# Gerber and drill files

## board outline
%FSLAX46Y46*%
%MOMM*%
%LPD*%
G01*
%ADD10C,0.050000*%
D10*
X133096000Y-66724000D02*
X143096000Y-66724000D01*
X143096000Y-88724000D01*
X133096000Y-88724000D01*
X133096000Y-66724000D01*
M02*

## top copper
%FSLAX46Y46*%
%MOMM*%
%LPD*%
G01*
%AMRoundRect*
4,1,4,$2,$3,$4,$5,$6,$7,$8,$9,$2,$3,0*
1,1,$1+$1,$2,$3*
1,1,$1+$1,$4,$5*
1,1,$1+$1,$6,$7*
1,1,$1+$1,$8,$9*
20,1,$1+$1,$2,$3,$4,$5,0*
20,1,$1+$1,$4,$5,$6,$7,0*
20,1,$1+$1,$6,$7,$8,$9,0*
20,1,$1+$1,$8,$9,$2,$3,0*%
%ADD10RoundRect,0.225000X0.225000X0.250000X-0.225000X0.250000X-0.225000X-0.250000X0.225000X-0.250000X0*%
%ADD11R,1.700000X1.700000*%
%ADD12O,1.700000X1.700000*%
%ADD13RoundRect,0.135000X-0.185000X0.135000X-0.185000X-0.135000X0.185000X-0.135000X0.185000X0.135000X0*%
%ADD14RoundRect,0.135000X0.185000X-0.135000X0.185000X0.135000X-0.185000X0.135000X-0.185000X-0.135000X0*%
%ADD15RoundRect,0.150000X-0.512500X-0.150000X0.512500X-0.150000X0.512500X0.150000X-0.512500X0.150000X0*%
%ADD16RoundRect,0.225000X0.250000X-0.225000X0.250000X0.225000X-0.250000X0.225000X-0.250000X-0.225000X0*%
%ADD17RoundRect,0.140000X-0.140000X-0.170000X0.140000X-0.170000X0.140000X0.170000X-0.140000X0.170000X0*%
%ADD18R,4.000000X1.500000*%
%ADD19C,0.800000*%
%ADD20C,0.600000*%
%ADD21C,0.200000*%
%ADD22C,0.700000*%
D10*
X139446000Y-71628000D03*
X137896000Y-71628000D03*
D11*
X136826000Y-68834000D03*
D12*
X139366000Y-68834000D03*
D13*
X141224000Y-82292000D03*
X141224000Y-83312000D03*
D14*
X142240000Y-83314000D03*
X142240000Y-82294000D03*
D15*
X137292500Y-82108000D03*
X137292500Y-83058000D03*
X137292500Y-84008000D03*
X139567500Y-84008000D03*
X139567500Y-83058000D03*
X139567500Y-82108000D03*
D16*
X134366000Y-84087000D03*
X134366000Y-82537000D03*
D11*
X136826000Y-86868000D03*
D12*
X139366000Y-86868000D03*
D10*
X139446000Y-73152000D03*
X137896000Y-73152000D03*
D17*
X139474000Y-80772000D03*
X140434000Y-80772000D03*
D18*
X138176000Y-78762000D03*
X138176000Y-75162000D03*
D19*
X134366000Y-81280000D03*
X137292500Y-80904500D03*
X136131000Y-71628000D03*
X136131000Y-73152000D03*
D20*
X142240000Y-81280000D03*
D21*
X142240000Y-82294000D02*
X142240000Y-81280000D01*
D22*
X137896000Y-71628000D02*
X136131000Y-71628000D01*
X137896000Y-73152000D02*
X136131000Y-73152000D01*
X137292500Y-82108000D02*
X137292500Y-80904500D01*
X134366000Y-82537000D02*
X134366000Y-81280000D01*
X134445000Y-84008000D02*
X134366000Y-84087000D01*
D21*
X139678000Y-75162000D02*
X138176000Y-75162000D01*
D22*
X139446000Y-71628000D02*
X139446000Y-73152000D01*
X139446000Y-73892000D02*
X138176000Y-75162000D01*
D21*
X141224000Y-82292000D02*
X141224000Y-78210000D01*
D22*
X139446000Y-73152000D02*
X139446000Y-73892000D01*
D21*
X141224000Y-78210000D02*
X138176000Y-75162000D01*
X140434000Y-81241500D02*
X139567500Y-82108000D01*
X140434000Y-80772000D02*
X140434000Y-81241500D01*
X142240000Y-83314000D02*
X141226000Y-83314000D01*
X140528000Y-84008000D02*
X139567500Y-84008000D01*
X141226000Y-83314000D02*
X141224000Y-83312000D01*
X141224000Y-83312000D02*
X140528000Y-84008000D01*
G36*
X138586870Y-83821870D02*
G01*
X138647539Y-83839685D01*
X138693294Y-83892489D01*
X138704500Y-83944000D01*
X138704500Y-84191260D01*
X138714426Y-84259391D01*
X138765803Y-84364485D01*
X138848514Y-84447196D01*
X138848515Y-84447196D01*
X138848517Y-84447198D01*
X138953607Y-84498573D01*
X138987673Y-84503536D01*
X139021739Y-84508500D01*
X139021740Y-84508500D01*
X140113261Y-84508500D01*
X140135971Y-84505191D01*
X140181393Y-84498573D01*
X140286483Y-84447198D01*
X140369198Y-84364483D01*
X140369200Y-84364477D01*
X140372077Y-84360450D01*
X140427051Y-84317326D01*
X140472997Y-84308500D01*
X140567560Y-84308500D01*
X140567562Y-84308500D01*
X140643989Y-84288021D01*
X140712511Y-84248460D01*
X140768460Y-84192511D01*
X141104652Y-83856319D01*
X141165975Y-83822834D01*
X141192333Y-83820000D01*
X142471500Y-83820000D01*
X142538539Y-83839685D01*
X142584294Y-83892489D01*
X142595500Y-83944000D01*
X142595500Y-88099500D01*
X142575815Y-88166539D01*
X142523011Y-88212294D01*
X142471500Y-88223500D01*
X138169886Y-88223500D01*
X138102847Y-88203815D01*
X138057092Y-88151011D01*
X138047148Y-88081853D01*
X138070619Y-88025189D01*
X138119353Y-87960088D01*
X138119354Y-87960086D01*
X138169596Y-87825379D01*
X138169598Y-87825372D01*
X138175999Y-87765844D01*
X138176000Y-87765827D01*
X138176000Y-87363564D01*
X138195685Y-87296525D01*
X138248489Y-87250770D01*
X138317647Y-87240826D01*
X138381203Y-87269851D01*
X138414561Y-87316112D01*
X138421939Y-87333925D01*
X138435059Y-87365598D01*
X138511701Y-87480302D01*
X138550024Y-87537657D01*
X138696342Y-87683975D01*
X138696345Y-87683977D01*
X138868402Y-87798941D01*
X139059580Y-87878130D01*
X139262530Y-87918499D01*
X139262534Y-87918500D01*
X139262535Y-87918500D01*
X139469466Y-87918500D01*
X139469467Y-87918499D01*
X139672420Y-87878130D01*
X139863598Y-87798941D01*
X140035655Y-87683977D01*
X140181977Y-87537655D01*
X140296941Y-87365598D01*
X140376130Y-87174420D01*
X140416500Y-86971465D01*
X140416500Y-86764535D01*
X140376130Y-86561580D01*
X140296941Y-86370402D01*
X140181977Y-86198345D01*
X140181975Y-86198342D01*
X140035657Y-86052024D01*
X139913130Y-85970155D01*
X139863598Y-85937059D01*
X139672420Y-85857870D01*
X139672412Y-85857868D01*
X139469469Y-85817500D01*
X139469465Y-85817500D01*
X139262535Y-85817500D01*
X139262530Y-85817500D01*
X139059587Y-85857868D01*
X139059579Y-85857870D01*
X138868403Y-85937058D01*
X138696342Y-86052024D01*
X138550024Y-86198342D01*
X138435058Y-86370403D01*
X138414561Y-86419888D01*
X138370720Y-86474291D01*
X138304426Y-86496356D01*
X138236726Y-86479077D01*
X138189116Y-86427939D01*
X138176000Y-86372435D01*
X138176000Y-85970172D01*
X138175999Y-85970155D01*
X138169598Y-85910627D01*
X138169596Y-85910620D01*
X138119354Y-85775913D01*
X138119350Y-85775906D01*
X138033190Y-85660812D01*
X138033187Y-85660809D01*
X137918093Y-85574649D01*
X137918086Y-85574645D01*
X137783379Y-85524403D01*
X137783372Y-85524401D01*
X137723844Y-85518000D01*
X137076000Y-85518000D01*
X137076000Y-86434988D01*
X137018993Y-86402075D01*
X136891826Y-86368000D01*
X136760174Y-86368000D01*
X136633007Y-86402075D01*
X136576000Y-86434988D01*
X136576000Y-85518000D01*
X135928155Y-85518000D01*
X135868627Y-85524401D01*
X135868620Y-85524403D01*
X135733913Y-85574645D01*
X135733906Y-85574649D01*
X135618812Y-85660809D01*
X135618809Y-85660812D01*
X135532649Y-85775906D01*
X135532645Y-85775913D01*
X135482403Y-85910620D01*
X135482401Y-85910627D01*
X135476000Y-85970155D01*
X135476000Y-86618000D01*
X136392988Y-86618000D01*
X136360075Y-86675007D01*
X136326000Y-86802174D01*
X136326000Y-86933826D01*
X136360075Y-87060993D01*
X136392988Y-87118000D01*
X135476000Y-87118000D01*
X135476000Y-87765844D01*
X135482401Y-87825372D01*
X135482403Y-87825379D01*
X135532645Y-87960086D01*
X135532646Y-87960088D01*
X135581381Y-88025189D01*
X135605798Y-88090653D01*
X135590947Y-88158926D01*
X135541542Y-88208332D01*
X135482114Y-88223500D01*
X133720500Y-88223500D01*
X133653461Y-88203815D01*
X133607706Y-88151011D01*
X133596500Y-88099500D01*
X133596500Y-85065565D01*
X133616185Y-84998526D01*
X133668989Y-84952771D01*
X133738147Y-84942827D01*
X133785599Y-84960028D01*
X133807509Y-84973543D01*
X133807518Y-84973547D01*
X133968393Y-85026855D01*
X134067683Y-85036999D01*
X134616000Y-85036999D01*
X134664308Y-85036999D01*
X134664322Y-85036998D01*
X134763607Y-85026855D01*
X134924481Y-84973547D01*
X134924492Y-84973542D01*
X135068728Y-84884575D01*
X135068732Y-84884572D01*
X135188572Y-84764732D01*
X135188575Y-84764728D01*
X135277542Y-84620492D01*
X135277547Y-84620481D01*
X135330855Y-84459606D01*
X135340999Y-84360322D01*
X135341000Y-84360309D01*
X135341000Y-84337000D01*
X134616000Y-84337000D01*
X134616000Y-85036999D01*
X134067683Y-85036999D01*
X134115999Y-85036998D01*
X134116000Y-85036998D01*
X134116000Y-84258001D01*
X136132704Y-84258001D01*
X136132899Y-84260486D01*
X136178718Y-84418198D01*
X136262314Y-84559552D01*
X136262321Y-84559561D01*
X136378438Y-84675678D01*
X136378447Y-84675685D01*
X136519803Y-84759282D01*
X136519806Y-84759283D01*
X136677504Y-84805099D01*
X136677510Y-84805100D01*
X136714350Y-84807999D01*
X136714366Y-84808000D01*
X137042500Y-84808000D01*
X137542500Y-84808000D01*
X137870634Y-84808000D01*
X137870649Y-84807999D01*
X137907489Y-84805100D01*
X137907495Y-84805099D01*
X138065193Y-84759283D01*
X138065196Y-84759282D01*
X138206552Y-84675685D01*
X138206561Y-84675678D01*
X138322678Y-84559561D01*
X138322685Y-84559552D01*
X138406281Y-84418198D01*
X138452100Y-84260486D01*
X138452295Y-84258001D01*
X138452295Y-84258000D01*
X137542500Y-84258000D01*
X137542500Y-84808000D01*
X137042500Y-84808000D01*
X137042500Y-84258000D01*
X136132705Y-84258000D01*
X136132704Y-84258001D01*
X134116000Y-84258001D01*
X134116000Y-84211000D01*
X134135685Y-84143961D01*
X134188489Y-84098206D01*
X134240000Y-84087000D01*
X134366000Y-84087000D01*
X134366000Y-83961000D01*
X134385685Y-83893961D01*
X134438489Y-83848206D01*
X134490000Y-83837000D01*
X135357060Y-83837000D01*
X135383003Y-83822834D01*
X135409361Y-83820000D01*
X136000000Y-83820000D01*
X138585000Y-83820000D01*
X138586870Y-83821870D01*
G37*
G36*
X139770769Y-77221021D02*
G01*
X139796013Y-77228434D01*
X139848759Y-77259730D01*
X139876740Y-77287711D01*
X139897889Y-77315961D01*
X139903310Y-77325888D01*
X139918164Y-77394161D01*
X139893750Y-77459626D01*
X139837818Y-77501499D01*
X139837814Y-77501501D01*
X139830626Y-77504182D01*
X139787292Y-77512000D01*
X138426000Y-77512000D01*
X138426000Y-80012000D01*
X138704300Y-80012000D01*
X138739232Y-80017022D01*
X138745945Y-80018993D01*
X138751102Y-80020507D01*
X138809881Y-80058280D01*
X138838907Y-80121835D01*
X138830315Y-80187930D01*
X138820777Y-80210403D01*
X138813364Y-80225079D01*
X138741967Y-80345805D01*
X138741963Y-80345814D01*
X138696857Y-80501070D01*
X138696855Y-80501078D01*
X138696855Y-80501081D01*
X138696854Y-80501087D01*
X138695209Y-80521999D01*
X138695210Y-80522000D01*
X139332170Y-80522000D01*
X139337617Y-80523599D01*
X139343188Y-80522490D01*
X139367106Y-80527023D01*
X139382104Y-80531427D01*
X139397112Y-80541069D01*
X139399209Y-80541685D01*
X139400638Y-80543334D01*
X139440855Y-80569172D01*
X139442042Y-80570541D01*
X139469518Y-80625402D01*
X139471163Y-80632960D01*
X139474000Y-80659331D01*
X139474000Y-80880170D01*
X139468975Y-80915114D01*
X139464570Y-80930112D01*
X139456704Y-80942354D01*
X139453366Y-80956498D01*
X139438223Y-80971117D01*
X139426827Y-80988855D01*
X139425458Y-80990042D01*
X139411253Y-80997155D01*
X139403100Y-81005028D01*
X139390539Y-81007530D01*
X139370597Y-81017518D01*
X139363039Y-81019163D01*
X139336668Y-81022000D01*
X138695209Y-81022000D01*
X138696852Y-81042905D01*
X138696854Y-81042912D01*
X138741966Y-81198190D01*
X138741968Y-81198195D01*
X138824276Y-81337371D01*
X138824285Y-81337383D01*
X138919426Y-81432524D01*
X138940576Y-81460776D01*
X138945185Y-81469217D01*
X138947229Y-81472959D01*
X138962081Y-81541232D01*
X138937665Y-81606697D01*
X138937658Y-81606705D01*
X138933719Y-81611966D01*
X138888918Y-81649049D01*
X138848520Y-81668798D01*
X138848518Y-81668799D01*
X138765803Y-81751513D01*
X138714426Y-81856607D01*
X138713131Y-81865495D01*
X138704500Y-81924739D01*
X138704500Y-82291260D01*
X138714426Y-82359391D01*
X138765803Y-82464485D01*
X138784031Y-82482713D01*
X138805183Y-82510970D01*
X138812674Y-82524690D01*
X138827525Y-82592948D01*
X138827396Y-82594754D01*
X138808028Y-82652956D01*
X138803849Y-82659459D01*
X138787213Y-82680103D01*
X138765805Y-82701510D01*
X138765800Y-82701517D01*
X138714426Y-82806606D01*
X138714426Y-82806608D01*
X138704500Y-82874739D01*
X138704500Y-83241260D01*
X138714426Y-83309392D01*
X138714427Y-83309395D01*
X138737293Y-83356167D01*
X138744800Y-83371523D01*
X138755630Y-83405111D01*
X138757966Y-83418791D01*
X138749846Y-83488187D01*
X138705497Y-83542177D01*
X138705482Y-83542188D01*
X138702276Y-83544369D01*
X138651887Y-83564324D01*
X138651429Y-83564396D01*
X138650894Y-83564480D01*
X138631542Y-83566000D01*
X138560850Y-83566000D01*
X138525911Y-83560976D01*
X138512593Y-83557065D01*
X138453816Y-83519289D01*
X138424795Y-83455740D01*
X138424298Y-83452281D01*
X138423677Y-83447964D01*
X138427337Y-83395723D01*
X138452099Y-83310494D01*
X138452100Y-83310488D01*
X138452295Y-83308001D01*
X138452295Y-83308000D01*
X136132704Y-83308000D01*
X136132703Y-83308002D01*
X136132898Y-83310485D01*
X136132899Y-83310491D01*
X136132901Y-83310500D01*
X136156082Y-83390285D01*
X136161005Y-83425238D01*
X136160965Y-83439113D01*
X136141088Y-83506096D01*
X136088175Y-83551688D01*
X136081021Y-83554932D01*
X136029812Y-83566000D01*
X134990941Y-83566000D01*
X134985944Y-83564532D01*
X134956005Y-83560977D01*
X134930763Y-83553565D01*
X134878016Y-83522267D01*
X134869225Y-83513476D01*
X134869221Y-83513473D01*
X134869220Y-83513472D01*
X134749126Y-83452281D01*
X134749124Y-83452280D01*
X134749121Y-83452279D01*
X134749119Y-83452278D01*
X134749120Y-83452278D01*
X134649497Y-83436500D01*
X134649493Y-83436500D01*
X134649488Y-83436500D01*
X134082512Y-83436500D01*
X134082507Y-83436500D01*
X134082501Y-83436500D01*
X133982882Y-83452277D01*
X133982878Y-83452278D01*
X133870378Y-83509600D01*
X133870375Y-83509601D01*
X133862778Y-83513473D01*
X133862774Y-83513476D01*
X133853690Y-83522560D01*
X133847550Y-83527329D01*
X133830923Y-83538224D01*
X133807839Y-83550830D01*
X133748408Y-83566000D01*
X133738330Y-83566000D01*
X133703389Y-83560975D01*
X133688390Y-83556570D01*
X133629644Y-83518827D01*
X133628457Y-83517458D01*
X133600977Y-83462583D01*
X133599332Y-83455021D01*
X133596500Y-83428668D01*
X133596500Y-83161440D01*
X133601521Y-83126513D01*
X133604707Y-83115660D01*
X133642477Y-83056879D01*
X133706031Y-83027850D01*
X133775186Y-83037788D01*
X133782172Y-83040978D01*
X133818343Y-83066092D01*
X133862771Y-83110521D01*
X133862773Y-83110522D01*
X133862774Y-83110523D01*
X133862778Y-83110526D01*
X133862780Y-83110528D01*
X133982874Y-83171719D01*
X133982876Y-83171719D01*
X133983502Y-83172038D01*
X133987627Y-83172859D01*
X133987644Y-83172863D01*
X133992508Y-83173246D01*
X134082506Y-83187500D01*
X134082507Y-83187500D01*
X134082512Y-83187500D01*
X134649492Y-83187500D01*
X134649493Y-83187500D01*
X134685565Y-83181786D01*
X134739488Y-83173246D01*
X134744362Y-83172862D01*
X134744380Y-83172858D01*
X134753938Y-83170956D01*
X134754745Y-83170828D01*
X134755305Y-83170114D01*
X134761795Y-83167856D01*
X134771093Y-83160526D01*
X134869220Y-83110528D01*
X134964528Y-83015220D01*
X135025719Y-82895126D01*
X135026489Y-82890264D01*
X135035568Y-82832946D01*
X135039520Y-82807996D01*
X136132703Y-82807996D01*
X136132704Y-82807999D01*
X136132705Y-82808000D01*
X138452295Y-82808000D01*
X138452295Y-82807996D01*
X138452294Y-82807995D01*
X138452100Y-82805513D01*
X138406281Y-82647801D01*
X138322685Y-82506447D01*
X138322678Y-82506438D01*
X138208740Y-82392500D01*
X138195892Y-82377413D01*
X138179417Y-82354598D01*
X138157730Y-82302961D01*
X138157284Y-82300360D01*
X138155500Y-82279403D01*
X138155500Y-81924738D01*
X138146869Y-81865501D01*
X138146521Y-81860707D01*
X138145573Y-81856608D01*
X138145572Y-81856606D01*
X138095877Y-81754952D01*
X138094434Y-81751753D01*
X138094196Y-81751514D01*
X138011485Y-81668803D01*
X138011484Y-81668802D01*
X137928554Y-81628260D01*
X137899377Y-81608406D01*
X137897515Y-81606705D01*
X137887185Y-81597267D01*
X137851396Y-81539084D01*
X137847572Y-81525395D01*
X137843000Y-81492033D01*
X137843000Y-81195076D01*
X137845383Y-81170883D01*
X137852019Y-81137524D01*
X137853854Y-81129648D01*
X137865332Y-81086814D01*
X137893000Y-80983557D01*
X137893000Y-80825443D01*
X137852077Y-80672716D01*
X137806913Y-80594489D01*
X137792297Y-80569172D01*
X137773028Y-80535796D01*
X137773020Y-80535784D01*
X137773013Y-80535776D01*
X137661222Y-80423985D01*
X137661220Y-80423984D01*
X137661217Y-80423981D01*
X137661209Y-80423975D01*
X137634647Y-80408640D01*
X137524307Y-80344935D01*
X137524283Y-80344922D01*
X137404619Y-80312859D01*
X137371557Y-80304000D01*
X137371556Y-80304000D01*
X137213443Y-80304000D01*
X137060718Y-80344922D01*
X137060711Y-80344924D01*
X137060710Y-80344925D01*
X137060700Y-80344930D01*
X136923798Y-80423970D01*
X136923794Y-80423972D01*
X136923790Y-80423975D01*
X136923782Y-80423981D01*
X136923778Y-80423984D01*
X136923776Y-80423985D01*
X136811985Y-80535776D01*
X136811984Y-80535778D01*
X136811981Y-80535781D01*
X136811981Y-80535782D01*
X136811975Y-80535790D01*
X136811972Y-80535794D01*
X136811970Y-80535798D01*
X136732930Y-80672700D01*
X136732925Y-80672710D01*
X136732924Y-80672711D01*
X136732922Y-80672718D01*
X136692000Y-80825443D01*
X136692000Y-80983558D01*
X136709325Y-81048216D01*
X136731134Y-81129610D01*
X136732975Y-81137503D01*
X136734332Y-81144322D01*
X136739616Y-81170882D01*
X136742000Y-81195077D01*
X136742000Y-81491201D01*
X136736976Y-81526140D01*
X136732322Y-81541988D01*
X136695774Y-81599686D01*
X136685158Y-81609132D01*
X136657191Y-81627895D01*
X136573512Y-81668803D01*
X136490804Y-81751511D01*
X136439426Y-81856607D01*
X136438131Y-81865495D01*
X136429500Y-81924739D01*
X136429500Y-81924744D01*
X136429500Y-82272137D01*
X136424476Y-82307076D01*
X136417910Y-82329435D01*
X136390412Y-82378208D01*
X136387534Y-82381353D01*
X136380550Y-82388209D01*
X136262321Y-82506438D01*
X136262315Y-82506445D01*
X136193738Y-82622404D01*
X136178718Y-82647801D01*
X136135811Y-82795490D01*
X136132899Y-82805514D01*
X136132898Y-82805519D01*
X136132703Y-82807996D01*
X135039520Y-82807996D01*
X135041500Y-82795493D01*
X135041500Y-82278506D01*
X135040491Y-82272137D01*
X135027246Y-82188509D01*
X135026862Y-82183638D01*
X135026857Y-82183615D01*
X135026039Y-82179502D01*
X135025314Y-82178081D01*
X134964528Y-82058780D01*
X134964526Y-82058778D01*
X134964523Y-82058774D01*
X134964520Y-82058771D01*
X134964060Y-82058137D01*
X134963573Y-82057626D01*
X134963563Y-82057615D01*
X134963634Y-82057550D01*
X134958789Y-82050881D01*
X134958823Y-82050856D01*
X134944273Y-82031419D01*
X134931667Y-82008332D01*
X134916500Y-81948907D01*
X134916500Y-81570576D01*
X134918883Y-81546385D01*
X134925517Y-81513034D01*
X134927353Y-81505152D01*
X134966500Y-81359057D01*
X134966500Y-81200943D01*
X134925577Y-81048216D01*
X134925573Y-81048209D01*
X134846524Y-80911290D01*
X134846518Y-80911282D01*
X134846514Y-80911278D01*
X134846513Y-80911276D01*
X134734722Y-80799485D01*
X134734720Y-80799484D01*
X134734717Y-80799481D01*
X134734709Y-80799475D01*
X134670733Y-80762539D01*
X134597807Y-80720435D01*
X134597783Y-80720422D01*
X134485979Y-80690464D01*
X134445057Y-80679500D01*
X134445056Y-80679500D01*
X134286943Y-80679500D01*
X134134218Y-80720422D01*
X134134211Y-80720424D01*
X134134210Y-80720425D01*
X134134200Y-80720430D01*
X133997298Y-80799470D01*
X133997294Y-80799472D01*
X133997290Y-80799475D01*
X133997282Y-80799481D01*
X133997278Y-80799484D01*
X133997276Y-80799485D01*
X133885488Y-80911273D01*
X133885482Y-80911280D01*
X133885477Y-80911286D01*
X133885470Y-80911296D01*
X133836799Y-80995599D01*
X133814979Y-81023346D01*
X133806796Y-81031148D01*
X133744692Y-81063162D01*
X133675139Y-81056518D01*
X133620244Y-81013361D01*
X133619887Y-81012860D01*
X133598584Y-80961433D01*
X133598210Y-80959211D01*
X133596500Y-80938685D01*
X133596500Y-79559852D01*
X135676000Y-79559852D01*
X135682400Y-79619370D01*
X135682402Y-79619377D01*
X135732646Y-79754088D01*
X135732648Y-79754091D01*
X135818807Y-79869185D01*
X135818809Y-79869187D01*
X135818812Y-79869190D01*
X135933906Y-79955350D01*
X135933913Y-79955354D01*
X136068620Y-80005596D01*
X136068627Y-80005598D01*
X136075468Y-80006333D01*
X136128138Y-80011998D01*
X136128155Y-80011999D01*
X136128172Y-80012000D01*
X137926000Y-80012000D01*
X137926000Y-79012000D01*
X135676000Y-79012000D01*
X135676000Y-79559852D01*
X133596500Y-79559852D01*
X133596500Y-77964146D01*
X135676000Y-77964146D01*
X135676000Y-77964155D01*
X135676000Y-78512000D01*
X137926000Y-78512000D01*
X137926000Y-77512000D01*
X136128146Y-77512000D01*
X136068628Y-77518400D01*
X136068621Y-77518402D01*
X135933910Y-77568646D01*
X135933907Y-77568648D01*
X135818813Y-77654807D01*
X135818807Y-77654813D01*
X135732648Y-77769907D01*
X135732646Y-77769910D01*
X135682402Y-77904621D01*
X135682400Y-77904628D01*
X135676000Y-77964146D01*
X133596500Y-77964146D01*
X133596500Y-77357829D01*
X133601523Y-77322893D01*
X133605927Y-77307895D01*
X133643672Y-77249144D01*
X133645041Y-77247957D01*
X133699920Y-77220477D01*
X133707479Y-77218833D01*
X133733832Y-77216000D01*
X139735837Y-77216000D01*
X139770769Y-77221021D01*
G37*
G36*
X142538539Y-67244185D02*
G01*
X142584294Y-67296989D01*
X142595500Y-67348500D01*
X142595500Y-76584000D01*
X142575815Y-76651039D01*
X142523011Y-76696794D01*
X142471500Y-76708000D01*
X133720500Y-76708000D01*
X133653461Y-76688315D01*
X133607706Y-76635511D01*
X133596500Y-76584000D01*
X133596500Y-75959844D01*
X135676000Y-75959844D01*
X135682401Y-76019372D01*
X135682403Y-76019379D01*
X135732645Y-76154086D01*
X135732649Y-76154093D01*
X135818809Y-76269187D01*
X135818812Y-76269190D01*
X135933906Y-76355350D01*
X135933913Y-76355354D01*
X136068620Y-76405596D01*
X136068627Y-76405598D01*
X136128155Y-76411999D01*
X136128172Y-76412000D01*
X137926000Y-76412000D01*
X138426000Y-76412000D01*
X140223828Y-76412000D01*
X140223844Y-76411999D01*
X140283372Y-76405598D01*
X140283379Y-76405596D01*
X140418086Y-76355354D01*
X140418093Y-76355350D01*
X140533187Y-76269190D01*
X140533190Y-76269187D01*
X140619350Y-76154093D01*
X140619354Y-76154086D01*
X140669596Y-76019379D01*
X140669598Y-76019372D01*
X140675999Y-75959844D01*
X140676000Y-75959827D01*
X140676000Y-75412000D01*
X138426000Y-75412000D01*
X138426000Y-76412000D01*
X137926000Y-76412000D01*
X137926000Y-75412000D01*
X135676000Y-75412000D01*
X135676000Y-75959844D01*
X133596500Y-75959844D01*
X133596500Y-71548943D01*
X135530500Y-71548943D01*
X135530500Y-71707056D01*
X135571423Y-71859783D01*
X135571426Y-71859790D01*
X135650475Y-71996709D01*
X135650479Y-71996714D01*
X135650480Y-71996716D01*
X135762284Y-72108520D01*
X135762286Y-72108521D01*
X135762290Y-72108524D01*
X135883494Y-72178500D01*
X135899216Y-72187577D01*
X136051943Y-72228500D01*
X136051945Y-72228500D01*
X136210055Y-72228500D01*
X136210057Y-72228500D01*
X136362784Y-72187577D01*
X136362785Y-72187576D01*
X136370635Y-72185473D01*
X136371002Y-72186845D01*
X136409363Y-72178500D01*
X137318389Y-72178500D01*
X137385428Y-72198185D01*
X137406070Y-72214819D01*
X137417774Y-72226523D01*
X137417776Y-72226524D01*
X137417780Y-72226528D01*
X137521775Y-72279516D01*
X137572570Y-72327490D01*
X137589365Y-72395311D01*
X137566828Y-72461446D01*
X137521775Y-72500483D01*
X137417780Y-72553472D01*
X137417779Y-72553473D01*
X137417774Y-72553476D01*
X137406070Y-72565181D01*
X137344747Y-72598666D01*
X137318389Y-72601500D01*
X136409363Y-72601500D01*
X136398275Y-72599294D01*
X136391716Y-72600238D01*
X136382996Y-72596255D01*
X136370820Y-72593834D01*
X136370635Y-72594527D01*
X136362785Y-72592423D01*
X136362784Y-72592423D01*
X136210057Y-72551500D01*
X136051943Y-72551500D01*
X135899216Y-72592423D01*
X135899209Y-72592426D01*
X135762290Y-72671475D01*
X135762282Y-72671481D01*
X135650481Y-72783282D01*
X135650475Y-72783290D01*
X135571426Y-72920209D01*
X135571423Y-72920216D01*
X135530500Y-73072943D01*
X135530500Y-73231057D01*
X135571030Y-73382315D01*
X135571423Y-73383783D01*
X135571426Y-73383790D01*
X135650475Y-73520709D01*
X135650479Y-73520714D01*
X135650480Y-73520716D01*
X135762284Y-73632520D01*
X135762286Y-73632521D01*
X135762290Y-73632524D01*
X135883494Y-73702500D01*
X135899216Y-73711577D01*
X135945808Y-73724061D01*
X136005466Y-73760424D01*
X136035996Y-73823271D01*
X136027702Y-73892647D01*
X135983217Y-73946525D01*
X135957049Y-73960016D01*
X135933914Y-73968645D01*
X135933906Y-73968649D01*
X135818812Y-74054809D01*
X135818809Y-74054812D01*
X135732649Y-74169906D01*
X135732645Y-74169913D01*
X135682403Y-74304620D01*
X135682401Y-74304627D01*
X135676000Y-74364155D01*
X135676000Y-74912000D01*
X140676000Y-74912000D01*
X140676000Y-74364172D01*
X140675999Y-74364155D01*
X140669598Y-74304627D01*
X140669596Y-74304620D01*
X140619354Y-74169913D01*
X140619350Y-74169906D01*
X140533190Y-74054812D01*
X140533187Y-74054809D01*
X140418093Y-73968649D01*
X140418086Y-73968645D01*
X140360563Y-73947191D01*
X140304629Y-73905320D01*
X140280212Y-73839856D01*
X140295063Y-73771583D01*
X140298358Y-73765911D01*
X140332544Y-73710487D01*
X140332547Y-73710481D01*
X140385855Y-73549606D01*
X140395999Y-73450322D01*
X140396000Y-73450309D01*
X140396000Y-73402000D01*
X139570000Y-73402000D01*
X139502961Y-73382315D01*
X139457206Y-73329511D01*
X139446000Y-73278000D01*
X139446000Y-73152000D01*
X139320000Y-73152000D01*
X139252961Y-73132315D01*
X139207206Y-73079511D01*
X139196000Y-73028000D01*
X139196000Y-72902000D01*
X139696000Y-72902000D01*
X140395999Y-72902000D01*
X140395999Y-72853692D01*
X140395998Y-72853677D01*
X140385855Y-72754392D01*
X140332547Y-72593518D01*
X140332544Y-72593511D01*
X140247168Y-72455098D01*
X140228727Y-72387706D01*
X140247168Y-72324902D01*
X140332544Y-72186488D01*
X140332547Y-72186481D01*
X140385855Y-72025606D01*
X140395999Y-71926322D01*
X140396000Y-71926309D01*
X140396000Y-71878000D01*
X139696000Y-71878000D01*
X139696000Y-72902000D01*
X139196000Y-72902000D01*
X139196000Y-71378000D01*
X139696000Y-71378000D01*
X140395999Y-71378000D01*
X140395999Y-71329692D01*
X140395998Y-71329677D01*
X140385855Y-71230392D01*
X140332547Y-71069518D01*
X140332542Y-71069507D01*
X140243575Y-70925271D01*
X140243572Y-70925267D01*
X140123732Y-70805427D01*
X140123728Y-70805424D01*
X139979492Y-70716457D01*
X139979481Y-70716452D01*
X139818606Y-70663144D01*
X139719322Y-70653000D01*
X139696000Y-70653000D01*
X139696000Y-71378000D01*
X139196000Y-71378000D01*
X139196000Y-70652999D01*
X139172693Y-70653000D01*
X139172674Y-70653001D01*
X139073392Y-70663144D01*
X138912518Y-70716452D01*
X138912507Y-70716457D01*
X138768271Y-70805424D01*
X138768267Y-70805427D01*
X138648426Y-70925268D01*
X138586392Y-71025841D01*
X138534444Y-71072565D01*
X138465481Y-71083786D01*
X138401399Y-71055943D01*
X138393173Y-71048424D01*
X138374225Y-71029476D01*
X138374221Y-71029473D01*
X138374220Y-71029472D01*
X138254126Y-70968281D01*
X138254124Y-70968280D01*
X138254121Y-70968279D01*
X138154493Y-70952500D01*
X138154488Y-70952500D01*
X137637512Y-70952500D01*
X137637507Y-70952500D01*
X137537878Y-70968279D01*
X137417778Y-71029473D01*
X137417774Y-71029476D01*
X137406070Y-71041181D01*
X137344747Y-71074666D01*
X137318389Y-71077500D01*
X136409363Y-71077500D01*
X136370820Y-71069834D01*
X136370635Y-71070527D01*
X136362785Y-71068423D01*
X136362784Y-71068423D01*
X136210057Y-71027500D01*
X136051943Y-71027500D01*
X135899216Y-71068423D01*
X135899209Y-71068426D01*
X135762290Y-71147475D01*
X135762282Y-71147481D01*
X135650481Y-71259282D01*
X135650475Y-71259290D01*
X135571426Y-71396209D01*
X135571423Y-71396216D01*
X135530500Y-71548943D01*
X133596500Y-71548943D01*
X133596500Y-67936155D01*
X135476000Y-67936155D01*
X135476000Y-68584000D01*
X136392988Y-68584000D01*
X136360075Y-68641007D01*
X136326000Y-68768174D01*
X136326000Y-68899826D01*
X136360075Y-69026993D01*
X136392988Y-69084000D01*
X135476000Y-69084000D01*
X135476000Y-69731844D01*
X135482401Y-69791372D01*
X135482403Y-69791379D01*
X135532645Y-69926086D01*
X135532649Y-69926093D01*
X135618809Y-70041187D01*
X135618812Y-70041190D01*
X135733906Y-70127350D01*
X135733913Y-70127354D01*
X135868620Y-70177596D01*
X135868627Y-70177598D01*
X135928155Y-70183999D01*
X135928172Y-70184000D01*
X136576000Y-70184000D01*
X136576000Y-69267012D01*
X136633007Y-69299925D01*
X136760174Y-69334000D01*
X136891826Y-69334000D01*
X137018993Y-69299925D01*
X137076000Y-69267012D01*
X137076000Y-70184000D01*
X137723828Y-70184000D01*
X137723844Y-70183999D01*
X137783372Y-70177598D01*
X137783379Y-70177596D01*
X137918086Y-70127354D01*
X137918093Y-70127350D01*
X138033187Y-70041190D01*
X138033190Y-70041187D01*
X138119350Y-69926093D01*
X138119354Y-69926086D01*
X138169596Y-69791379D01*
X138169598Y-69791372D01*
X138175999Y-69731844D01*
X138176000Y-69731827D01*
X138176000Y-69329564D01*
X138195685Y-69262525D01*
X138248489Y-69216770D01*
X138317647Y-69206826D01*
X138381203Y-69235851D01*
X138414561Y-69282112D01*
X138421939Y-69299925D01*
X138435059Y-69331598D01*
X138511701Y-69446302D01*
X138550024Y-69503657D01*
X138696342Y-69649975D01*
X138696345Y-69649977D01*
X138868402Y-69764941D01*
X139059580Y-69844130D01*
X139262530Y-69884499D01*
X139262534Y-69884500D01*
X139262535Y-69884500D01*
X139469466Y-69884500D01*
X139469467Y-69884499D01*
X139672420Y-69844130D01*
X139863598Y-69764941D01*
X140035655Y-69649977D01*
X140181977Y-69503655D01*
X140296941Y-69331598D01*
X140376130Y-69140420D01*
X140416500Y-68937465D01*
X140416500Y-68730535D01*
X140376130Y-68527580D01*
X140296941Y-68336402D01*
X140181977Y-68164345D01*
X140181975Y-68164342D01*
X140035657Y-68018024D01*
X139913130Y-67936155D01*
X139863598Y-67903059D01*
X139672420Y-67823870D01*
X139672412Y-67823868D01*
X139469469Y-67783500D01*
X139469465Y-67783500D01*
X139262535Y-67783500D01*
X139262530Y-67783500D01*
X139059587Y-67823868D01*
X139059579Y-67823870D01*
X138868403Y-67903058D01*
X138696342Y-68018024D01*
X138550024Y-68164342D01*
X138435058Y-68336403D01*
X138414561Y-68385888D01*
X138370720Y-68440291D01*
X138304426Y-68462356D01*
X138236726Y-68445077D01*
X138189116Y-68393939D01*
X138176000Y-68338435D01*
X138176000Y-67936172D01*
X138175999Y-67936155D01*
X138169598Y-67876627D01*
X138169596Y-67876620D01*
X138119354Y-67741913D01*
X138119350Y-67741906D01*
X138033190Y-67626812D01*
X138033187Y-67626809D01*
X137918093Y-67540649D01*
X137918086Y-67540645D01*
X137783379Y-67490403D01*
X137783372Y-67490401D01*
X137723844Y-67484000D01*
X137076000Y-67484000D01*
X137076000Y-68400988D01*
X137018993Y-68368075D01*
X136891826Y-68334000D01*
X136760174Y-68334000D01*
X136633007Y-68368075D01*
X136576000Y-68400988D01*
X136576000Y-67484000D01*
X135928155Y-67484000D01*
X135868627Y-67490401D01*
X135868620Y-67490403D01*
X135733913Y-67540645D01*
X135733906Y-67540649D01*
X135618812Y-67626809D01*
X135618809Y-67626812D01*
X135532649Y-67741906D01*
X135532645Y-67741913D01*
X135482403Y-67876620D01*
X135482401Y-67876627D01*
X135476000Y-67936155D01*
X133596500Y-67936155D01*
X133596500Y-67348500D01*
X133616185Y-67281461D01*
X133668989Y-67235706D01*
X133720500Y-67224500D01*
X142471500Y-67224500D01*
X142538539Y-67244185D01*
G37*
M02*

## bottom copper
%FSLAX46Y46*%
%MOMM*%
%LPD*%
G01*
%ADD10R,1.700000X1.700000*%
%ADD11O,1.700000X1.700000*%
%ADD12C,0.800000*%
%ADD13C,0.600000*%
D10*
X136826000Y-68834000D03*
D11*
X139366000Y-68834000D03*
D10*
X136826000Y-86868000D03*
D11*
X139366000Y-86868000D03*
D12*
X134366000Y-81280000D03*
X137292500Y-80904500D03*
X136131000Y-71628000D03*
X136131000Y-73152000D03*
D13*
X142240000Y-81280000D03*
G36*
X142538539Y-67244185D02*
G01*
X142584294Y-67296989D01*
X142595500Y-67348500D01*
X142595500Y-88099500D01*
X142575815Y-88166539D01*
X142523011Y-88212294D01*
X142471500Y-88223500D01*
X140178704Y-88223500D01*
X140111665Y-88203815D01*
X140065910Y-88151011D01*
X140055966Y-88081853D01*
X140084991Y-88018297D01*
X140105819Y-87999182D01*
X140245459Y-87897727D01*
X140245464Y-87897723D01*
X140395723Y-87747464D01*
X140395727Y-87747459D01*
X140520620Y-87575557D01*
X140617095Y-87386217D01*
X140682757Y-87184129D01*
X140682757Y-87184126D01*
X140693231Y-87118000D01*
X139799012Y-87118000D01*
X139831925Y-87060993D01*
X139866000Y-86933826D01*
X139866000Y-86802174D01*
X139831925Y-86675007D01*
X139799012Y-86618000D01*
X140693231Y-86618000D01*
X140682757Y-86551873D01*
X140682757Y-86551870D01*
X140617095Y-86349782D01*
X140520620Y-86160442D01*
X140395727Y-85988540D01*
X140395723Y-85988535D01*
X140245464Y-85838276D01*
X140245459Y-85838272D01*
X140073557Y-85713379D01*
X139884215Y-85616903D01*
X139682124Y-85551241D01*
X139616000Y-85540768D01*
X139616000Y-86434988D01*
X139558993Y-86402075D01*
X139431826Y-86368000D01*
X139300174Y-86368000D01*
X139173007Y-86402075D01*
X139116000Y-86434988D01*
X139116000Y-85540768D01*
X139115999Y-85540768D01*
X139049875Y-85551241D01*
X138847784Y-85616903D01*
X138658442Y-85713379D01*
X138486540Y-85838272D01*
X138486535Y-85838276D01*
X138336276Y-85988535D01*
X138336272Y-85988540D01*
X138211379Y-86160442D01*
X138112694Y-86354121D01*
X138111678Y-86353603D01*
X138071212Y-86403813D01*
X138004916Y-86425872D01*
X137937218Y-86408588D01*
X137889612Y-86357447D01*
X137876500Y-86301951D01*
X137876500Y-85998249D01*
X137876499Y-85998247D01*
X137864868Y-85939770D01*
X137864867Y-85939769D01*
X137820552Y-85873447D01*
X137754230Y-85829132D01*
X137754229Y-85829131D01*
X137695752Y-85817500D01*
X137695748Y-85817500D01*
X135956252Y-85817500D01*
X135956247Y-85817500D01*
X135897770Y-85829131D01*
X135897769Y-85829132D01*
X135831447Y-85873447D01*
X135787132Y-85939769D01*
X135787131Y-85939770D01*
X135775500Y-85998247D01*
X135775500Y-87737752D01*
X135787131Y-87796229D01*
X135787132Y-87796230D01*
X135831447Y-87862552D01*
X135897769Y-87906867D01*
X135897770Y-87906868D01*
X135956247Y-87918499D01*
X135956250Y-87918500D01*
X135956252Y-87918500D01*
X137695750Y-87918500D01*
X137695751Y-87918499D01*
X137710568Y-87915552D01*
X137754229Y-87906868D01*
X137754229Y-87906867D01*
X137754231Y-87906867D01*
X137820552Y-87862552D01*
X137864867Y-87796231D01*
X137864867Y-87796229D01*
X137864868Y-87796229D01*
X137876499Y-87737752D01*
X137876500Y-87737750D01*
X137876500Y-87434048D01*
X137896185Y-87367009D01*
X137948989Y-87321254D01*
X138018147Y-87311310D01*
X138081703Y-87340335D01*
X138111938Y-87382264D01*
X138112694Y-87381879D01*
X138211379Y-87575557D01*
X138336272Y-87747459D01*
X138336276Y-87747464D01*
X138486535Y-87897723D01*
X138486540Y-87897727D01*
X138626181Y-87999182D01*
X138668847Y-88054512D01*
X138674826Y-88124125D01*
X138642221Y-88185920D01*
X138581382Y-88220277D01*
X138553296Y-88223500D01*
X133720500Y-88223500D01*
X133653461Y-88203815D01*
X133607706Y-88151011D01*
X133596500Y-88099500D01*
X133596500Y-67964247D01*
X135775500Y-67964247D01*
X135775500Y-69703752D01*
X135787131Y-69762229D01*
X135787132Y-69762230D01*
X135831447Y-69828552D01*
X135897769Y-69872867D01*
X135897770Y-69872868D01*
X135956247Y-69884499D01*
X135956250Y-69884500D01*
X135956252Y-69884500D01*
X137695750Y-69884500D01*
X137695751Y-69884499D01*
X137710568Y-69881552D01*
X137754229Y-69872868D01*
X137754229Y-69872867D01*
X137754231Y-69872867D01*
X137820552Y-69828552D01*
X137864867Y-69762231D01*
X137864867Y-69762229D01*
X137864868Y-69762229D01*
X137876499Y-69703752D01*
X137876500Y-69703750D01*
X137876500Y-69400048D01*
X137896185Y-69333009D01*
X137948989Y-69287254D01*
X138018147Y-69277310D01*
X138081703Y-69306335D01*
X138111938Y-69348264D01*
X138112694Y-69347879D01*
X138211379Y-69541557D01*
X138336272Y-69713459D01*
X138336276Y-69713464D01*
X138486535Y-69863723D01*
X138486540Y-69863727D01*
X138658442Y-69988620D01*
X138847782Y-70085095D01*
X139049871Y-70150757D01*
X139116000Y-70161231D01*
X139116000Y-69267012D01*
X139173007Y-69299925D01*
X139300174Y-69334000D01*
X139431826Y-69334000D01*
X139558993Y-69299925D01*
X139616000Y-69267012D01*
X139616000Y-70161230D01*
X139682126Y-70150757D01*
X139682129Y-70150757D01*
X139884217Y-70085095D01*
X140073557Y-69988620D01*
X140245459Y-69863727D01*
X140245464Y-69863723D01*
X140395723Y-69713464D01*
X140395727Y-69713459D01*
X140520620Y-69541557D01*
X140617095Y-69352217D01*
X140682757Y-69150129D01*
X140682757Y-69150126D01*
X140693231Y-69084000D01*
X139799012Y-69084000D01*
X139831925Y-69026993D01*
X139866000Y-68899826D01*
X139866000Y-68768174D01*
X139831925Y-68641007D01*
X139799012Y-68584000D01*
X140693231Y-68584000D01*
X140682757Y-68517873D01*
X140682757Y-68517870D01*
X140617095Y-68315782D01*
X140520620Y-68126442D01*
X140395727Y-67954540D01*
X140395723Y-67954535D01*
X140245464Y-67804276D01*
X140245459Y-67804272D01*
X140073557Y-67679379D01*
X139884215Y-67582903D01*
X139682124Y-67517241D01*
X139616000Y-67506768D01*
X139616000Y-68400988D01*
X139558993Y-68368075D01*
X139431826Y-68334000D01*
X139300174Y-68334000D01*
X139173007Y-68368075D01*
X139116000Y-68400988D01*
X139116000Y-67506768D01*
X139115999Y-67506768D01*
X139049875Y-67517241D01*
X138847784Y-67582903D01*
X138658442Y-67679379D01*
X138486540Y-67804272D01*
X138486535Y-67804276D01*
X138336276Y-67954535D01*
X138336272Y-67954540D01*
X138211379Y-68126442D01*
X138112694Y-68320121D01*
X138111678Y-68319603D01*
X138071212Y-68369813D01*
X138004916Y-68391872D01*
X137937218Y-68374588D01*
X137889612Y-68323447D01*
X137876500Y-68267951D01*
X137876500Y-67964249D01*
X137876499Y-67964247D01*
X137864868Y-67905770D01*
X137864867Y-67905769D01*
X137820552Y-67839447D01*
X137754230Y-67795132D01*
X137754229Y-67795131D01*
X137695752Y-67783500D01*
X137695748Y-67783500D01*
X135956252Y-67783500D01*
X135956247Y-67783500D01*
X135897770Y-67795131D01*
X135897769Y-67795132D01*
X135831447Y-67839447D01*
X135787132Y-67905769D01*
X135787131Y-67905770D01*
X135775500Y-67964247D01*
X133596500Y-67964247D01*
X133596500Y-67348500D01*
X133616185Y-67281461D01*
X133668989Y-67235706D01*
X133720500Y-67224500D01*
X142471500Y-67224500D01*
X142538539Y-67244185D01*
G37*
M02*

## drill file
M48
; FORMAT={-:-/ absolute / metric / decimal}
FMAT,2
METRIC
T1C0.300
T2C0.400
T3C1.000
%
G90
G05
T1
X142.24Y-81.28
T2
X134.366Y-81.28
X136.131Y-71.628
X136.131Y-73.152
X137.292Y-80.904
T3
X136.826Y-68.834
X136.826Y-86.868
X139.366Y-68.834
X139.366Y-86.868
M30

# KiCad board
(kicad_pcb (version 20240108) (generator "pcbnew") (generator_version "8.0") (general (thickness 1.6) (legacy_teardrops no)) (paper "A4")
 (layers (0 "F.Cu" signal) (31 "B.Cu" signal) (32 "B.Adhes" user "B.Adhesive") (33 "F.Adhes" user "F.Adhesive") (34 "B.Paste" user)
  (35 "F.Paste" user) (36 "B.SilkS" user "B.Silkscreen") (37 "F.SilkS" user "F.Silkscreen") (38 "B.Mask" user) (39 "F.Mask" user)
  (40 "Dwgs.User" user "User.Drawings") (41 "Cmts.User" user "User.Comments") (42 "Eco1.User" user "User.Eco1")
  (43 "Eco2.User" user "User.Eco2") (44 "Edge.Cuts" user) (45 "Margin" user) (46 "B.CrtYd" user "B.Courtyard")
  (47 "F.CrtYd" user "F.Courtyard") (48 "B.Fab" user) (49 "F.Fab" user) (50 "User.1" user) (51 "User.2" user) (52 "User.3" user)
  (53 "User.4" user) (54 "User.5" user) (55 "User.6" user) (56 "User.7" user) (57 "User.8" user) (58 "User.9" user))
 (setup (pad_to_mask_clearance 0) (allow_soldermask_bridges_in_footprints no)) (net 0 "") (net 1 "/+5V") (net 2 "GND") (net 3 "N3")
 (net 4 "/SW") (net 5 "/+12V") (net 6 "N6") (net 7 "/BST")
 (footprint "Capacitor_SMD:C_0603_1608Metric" (layer "F.Cu") (at 138.671 71.628 180)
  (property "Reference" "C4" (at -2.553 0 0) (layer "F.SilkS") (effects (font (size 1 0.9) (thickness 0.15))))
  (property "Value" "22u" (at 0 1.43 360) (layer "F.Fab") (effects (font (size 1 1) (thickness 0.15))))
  (pad "1" smd roundrect (at -0.775 0 180) (size 0.9 0.95) (layers "F.Cu" "F.Paste" "F.Mask") (roundrect_rratio 0.25) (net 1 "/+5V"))
  (pad "2" smd roundrect (at 0.775 0 180) (size 0.9 0.95) (layers "F.Cu" "F.Paste" "F.Mask") (roundrect_rratio 0.25) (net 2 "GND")))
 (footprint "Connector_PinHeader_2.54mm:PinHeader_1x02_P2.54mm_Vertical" (layer "F.Cu") (at 136.826 68.834 90)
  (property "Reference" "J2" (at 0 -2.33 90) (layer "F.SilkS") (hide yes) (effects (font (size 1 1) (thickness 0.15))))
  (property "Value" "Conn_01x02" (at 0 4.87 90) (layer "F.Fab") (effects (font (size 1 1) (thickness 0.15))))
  (pad "1" thru_hole rect (at 0 0 90) (size 1.7 1.7) (drill 1) (layers "*.Cu" "*.Mask") (remove_unused_layers no) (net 1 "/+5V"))
  (pad "2" thru_hole oval (at 0 2.54 90) (size 1.7 1.7) (drill 1) (layers "*.Cu" "*.Mask") (remove_unused_layers no) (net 2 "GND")))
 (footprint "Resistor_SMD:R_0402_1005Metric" (layer "F.Cu") (at 141.224 82.802 -90)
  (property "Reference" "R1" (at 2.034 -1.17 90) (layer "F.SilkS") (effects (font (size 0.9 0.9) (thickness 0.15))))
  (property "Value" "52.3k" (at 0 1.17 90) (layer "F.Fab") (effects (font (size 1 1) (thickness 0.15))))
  (pad "1" smd roundrect (at -0.51 0 270) (size 0.54 0.64) (layers "F.Cu" "F.Paste" "F.Mask") (roundrect_rratio 0.25) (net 1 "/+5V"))
  (pad "2" smd roundrect (at 0.51 0 270) (size 0.54 0.64) (layers "F.Cu" "F.Paste" "F.Mask") (roundrect_rratio 0.25) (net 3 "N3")))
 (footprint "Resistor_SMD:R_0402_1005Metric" (layer "F.Cu") (at 142.24 82.804 90)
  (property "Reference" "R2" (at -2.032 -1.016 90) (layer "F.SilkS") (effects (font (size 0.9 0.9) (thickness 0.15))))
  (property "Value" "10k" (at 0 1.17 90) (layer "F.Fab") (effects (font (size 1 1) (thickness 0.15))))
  (pad "1" smd roundrect (at -0.51 0 90) (size 0.54 0.64) (layers "F.Cu" "F.Paste" "F.Mask") (roundrect_rratio 0.25) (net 3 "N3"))
  (pad "2" smd roundrect (at 0.51 0 90) (size 0.54 0.64) (layers "F.Cu" "F.Paste" "F.Mask") (roundrect_rratio 0.25) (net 2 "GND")))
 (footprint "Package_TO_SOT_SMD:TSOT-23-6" (layer "F.Cu") (at 138.43 83.058)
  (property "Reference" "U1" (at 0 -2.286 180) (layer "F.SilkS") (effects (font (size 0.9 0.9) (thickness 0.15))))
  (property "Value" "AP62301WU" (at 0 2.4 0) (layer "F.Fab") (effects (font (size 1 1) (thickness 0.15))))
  (pad "1" smd roundrect (at -1.1375 -0.95) (size 1.325 0.6) (layers "F.Cu" "F.Paste" "F.Mask") (roundrect_rratio 0.25) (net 2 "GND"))
  (pad "2" smd roundrect (at -1.1375 0) (size 1.325 0.6) (layers "F.Cu" "F.Paste" "F.Mask") (roundrect_rratio 0.25) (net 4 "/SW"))
  (pad "3" smd roundrect (at -1.1375 0.95) (size 1.325 0.6) (layers "F.Cu" "F.Paste" "F.Mask") (roundrect_rratio 0.25) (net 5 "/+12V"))
  (pad "4" smd roundrect (at 1.1375 0.95) (size 1.325 0.6) (layers "F.Cu" "F.Paste" "F.Mask") (roundrect_rratio 0.25) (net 3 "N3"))
  (pad "5" smd roundrect (at 1.1375 0) (size 1.325 0.6) (layers "F.Cu" "F.Paste" "F.Mask") (roundrect_rratio 0.25) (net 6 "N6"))
  (pad "6" smd roundrect (at 1.1375 -0.95) (size 1.325 0.6) (layers "F.Cu" "F.Paste" "F.Mask") (roundrect_rratio 0.25) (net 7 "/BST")))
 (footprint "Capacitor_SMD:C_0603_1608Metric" (layer "F.Cu") (at 134.366 83.312 90)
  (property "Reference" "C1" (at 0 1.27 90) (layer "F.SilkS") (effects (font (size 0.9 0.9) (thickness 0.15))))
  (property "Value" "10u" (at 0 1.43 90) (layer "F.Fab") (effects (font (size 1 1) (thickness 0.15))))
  (pad "1" smd roundrect (at -0.775 0 90) (size 0.9 0.95) (layers "F.Cu" "F.Paste" "F.Mask") (roundrect_rratio 0.25) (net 5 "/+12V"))
  (pad "2" smd roundrect (at 0.775 0 90) (size 0.9 0.95) (layers "F.Cu" "F.Paste" "F.Mask") (roundrect_rratio 0.25) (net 2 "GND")))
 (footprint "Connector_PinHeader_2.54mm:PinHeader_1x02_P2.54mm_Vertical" (layer "F.Cu") (at 136.826 86.868 90)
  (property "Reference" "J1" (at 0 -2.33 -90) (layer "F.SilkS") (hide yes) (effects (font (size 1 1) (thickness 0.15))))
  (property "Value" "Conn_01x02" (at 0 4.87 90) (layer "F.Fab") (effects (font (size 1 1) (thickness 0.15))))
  (pad "1" thru_hole rect (at 0 0 90) (size 1.7 1.7) (drill 1) (layers "*.Cu" "*.Mask") (remove_unused_layers no) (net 5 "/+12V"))
  (pad "2" thru_hole oval (at 0 2.54 90) (size 1.7 1.7) (drill 1) (layers "*.Cu" "*.Mask") (remove_unused_layers no) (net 2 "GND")))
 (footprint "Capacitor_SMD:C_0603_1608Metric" (layer "F.Cu") (at 138.671 73.152 180)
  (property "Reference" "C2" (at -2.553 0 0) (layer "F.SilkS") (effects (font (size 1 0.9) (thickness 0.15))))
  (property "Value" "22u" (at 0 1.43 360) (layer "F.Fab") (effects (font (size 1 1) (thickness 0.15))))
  (pad "1" smd roundrect (at -0.775 0 180) (size 0.9 0.95) (layers "F.Cu" "F.Paste" "F.Mask") (roundrect_rratio 0.25) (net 1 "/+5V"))
  (pad "2" smd roundrect (at 0.775 0 180) (size 0.9 0.95) (layers "F.Cu" "F.Paste" "F.Mask") (roundrect_rratio 0.25) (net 2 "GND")))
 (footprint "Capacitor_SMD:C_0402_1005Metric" (layer "F.Cu") (at 139.954 80.772)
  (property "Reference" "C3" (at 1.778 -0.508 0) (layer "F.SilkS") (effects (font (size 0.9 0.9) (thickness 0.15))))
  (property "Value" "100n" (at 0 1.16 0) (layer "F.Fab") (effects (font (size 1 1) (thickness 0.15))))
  (pad "1" smd roundrect (at -0.48 0) (size 0.56 0.62) (layers "F.Cu" "F.Paste" "F.Mask") (roundrect_rratio 0.25) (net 4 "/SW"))
  (pad "2" smd roundrect (at 0.48 0) (size 0.56 0.62) (layers "F.Cu" "F.Paste" "F.Mask") (roundrect_rratio 0.25) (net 7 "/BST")))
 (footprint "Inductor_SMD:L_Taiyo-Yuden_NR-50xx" (layer "F.Cu") (at 138.176 76.962 90)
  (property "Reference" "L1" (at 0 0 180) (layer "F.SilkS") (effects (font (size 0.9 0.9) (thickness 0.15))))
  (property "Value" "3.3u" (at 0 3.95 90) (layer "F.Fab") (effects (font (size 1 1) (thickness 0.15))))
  (pad "1" smd rect (at -1.8 0 90) (size 1.5 4) (layers "F.Cu" "F.Paste" "F.Mask") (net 4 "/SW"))
  (pad "2" smd rect (at 1.8 0 90) (size 1.5 4) (layers "F.Cu" "F.Paste" "F.Mask") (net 1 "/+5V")))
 (gr_rect (start 133.096 66.724) (end 143.096 88.724) (stroke (width 0.05) (type default)) (fill none) (layer "Edge.Cuts"))
 (segment (start 142.24 82.294) (end 142.24 81.28) (width 0.2) (layer "F.Cu") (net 2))
 (segment (start 137.896 71.628) (end 136.131 71.628) (width 0.7) (layer "F.Cu") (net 2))
 (segment (start 137.896 73.152) (end 136.131 73.152) (width 0.7) (layer "F.Cu") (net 2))
 (segment (start 137.2925 82.108) (end 137.2925 80.9045) (width 0.7) (layer "F.Cu") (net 2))
 (segment (start 134.366 82.537) (end 134.366 81.28) (width 0.7) (layer "F.Cu") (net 2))
 (via (at 134.366 81.28) (size 0.8) (drill 0.4) (layers "F.Cu" "B.Cu") (free yes) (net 2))
 (via (at 137.2925 80.9045) (size 0.8) (drill 0.4) (layers "F.Cu" "B.Cu") (free yes) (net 2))
 (via (at 136.131 71.628) (size 0.8) (drill 0.4) (layers "F.Cu" "B.Cu") (free yes) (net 2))
 (via (at 136.131 73.152) (size 0.8) (drill 0.4) (layers "F.Cu" "B.Cu") (free yes) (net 2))
 (via (at 142.24 81.28) (size 0.6) (drill 0.3) (layers "F.Cu" "B.Cu") (free yes) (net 2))
 (segment (start 134.445 84.008) (end 134.366 84.087) (width 0.7) (layer "F.Cu") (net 5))
 (segment (start 139.678 75.162) (end 138.176 75.162) (width 0.2) (layer "F.Cu") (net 1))
 (segment (start 139.446 71.628) (end 139.446 73.152) (width 0.7) (layer "F.Cu") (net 1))
 (segment (start 139.446 73.892) (end 138.176 75.162) (width 0.7) (layer "F.Cu") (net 1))
 (segment (start 141.224 82.292) (end 141.224 78.21) (width 0.2) (layer "F.Cu") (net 1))
 (segment (start 139.446 73.152) (end 139.446 73.892) (width 0.7) (layer "F.Cu") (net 1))
 (segment (start 141.224 78.21) (end 138.176 75.162) (width 0.2) (layer "F.Cu") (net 1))
 (segment (start 140.434 81.2415) (end 139.5675 82.108) (width 0.2) (layer "F.Cu") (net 7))
 (segment (start 140.434 80.772) (end 140.434 81.2415) (width 0.2) (layer "F.Cu") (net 7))
 (segment (start 142.24 83.314) (end 141.226 83.314) (width 0.2) (layer "F.Cu") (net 3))
 (segment (start 140.528 84.008) (end 139.5675 84.008) (width 0.2) (layer "F.Cu") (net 3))
 (segment (start 141.226 83.314) (end 141.224 83.312) (width 0.2) (layer "F.Cu") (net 3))
 (segment (start 141.224 83.312) (end 140.528 84.008) (width 0.2) (layer "F.Cu") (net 3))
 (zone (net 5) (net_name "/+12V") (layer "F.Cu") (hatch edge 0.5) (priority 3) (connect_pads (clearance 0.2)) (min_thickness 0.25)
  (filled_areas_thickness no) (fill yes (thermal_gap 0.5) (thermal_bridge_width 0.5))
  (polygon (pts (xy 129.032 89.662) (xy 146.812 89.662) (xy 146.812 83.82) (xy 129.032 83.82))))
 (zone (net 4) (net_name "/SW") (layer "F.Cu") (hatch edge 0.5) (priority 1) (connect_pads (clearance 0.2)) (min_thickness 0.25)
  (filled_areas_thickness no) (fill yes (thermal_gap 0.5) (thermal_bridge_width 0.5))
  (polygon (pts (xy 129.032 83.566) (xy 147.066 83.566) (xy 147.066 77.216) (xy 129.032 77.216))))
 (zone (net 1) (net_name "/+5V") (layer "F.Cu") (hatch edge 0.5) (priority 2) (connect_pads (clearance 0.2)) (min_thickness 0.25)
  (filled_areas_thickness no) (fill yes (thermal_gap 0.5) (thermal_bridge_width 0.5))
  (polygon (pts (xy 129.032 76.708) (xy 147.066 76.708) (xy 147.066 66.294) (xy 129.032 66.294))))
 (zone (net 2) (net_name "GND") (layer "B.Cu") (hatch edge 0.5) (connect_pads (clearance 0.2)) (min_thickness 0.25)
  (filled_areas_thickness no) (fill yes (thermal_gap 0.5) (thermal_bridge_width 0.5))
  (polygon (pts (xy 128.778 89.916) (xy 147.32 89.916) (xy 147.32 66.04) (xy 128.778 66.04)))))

